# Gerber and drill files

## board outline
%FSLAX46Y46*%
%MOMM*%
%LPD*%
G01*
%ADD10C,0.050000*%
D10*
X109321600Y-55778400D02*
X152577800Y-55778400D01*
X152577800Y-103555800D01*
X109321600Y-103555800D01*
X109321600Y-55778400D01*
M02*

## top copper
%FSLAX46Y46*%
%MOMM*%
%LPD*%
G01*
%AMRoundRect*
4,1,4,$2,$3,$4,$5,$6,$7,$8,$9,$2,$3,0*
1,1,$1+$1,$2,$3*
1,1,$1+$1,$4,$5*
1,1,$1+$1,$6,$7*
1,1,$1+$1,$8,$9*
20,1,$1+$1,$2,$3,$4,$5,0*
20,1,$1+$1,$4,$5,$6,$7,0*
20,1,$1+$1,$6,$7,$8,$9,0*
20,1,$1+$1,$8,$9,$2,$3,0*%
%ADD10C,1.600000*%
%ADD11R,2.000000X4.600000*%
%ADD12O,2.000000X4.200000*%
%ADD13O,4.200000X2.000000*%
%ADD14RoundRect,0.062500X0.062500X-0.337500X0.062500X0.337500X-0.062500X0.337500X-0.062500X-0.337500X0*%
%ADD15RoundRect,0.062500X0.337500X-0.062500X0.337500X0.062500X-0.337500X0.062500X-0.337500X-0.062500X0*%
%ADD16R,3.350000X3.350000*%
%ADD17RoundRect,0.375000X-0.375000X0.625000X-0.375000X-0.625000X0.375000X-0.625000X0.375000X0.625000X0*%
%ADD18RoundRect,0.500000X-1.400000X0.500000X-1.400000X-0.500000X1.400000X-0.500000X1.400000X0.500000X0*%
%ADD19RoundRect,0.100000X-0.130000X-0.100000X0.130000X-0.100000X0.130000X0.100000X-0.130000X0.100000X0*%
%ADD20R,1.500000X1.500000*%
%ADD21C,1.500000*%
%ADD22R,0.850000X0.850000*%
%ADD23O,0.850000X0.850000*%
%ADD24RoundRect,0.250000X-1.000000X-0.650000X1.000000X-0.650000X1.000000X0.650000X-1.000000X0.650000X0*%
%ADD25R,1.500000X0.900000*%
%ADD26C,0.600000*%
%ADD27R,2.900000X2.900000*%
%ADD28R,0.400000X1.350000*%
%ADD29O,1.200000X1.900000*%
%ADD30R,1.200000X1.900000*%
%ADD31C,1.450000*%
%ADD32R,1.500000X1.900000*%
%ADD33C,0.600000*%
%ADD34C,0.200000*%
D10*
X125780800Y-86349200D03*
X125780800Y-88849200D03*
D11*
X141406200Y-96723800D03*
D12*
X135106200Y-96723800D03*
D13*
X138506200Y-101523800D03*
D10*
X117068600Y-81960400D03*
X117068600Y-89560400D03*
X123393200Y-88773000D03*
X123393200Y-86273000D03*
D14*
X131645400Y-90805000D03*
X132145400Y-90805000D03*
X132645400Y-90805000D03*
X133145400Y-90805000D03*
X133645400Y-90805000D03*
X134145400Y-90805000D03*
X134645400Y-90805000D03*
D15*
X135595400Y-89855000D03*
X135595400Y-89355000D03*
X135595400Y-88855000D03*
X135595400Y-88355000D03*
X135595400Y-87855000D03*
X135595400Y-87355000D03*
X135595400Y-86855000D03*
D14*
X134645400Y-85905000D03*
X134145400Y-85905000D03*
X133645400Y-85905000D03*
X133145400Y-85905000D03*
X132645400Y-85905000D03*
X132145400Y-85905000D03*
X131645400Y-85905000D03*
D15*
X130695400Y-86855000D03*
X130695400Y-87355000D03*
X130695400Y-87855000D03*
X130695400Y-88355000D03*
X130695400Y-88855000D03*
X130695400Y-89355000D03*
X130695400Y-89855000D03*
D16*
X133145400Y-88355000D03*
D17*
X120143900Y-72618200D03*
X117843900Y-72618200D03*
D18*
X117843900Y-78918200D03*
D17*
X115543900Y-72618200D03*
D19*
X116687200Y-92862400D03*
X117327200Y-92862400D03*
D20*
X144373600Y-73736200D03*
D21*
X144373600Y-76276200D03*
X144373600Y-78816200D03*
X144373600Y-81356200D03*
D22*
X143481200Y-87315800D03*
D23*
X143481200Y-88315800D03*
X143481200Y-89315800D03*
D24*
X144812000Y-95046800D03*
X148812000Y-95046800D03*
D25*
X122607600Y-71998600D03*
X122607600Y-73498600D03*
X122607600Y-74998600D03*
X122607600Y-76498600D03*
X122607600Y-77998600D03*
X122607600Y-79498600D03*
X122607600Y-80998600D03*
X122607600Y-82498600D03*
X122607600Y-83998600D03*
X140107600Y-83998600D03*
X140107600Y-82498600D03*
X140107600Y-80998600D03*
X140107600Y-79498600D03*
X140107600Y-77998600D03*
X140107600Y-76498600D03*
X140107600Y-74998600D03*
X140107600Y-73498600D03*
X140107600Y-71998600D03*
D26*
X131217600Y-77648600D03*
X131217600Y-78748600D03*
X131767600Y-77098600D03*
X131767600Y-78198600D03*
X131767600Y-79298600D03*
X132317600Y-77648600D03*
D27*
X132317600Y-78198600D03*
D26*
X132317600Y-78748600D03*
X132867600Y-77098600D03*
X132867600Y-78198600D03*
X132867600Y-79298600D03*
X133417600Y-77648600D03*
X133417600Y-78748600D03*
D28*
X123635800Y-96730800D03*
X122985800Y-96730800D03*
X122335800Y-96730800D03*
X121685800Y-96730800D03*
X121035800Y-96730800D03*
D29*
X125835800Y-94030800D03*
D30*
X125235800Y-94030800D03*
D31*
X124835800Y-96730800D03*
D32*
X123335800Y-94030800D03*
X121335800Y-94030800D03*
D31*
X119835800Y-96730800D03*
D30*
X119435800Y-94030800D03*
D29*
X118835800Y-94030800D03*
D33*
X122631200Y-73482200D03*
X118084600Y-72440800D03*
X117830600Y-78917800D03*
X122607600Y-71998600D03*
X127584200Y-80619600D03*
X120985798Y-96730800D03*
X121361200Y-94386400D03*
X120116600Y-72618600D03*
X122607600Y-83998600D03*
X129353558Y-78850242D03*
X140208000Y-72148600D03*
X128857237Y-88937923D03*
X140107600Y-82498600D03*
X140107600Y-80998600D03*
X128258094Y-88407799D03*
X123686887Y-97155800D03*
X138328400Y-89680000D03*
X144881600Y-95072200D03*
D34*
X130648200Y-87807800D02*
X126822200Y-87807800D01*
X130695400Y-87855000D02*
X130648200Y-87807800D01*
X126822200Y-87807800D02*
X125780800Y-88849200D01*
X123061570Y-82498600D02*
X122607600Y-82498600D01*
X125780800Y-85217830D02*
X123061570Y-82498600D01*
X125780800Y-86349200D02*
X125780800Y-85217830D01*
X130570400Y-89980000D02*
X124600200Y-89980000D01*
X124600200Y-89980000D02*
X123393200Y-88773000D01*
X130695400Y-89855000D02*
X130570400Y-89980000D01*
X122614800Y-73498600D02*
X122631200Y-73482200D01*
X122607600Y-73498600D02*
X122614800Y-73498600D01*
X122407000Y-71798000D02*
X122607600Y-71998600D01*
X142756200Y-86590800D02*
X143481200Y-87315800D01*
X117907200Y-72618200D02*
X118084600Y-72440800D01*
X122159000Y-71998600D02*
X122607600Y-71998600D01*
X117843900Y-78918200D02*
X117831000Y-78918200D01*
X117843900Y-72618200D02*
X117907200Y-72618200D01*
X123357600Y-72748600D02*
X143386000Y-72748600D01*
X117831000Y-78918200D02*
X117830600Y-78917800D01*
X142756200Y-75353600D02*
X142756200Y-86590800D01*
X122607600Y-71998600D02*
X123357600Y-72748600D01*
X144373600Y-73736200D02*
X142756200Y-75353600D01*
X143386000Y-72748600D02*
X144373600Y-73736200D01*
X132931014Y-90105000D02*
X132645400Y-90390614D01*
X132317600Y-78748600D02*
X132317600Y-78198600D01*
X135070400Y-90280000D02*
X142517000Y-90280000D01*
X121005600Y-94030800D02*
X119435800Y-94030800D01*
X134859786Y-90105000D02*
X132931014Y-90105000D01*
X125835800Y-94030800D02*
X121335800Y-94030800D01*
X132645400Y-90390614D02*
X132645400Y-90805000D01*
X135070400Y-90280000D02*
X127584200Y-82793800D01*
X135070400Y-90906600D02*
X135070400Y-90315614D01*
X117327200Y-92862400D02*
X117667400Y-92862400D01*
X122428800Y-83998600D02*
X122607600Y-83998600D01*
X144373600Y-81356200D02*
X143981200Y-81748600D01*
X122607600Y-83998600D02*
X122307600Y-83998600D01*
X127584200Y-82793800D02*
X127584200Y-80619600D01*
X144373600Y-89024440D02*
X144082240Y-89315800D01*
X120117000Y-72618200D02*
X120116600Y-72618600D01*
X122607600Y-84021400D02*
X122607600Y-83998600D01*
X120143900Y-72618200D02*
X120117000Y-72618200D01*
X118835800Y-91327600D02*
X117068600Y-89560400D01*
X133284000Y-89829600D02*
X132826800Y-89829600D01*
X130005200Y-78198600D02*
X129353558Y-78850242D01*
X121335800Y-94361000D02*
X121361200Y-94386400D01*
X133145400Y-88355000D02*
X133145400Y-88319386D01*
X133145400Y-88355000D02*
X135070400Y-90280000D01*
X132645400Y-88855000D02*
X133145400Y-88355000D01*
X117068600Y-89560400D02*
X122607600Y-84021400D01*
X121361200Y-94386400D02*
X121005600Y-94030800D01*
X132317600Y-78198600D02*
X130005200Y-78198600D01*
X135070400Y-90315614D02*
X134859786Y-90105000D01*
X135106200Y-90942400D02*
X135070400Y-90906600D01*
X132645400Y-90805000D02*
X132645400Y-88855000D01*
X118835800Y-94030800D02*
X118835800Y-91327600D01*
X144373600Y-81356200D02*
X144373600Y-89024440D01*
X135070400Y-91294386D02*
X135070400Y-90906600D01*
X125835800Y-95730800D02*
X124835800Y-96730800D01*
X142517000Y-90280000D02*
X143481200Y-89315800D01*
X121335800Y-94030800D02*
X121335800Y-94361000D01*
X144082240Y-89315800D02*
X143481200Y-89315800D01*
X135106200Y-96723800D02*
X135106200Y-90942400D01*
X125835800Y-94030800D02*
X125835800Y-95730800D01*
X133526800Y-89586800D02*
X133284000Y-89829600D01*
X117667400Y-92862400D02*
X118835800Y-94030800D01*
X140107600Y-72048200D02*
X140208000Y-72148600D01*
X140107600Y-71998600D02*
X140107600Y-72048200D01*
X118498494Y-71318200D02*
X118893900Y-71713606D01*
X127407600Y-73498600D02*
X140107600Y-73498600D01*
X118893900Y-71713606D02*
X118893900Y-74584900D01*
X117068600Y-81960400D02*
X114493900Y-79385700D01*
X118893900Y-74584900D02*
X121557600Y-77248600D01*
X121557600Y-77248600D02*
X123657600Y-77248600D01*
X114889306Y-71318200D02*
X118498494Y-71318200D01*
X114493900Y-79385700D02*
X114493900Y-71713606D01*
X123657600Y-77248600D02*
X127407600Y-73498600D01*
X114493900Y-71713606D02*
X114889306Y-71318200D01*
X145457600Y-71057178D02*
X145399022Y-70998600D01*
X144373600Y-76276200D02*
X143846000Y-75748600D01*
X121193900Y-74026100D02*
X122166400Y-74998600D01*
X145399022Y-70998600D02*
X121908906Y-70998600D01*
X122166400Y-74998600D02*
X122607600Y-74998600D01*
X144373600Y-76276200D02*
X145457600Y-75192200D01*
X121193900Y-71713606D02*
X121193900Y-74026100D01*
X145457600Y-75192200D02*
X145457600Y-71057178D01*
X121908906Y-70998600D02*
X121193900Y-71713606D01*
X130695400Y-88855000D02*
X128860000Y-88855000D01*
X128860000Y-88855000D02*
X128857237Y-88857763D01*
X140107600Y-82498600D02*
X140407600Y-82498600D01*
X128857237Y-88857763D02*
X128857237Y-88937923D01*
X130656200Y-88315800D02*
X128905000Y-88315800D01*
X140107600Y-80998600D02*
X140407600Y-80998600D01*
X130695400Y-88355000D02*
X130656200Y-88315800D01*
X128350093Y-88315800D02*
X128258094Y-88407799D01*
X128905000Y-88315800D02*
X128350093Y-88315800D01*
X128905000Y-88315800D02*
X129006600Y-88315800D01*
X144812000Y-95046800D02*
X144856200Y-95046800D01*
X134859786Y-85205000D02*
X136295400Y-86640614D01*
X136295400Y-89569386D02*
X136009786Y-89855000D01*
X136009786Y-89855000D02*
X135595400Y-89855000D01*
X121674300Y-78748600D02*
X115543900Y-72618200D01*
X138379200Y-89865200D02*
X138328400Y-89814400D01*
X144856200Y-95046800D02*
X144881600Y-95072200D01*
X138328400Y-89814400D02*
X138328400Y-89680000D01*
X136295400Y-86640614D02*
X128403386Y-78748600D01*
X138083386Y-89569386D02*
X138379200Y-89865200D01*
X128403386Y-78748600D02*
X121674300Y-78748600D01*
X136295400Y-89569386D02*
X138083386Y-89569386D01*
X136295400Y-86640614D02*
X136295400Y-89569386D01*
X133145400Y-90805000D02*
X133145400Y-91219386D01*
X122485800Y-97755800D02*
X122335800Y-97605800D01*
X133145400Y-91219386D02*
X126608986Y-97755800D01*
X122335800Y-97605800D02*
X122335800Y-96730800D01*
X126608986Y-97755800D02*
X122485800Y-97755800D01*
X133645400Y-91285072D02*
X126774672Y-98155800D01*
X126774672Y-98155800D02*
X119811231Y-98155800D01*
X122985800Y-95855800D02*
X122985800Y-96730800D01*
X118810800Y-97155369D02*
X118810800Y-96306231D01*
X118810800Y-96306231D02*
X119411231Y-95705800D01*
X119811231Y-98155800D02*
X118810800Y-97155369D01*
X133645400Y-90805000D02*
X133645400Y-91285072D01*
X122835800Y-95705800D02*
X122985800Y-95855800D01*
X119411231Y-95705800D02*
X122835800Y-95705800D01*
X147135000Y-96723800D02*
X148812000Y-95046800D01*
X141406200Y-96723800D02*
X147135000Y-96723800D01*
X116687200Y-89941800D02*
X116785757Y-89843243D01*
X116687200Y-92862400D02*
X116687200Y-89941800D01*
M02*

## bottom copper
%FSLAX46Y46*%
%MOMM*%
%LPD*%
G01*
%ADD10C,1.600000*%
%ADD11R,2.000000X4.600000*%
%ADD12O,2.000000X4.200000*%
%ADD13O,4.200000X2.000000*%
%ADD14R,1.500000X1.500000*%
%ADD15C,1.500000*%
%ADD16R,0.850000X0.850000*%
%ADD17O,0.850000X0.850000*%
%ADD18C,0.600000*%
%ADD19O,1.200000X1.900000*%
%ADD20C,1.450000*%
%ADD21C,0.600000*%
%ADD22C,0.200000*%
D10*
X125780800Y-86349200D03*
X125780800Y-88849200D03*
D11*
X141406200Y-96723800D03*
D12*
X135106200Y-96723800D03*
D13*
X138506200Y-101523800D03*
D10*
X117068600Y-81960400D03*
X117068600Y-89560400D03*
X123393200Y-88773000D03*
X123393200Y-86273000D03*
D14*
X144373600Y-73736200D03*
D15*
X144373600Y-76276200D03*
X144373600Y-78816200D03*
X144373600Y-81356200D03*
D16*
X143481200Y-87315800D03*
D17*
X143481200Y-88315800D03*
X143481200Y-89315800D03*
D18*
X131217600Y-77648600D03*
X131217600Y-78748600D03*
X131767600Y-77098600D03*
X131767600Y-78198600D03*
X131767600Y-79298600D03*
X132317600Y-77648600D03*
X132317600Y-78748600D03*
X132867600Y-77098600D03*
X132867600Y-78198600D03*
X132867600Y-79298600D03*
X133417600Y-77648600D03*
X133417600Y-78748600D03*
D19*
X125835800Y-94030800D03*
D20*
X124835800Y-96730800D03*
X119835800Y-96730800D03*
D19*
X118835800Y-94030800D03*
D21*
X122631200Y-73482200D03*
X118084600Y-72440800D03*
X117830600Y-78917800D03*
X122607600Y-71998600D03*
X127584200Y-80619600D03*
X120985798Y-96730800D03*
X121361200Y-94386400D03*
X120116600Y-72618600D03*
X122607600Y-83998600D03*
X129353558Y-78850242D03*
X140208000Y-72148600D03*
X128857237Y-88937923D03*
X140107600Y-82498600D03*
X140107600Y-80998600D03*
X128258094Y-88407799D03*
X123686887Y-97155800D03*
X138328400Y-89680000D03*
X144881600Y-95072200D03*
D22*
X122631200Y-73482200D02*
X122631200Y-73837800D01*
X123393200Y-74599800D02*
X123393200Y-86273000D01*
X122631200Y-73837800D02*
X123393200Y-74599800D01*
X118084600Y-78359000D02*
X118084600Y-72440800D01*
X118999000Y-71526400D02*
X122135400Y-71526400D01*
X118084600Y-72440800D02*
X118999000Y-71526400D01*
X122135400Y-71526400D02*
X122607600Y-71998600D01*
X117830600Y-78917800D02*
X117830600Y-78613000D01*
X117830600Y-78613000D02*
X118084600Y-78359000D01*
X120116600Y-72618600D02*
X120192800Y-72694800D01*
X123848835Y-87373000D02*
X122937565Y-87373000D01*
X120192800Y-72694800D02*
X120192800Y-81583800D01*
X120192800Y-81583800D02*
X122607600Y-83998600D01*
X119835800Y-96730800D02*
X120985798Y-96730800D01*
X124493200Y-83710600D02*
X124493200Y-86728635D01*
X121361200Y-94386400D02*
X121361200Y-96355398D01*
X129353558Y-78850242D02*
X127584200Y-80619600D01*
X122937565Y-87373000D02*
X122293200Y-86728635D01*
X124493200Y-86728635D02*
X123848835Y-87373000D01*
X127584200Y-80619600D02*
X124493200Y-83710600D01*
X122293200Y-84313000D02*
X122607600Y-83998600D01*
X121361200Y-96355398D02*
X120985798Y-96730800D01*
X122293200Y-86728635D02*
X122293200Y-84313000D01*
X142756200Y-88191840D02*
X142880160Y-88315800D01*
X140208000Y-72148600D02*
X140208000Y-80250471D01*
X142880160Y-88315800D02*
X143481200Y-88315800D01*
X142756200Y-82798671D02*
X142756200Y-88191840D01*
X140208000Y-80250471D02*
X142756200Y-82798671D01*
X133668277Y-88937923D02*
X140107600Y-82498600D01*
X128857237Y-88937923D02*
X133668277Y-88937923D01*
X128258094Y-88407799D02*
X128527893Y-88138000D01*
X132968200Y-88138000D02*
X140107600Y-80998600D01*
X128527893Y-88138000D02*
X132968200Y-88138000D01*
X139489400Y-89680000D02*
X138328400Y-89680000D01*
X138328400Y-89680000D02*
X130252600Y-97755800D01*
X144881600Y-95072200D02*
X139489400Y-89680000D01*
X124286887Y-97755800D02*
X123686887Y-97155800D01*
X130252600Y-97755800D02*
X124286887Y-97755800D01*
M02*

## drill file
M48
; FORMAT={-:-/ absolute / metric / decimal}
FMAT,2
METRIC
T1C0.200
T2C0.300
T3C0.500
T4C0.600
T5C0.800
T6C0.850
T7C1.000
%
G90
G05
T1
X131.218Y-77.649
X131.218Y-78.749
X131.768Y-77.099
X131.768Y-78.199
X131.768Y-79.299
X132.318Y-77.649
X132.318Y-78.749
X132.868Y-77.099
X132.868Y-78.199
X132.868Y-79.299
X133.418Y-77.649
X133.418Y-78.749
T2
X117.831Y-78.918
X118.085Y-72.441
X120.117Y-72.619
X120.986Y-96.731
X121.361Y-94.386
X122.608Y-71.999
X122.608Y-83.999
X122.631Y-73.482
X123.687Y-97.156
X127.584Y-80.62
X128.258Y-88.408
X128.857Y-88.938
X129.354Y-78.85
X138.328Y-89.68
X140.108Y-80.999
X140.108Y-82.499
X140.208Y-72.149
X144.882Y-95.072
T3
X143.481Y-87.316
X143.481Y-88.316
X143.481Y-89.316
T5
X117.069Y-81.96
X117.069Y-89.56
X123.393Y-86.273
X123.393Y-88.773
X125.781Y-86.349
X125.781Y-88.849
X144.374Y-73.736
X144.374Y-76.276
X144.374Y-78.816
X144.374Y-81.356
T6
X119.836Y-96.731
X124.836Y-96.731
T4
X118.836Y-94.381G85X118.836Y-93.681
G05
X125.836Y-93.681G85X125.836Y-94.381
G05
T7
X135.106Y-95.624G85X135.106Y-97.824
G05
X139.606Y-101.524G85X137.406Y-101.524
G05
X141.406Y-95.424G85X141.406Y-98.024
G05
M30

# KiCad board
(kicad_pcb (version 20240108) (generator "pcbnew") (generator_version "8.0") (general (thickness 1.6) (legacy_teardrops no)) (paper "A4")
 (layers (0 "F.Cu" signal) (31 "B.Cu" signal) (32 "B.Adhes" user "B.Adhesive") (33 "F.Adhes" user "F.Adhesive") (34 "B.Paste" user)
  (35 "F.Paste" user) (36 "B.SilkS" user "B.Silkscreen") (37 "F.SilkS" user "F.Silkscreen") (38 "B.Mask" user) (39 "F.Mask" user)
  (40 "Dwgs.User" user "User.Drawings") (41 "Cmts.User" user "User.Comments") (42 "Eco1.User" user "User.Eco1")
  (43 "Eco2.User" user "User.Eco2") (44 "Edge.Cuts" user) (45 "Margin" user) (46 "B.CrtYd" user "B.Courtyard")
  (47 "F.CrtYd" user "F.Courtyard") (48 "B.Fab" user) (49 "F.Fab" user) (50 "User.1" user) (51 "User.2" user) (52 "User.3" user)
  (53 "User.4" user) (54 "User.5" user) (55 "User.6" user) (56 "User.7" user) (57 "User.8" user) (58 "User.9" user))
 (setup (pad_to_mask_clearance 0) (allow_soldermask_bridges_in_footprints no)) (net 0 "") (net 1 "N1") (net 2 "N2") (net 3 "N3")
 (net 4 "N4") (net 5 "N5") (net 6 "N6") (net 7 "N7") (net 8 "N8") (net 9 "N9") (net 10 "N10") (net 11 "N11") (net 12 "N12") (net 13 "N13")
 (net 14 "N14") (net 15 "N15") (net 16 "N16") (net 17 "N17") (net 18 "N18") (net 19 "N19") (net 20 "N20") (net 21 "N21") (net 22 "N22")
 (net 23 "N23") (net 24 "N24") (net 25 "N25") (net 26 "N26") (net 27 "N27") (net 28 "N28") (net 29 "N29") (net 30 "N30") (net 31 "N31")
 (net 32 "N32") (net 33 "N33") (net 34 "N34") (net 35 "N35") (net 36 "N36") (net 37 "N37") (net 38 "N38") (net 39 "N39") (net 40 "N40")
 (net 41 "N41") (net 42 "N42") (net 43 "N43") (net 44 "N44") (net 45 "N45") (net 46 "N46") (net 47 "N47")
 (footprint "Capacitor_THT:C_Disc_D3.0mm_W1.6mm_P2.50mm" (layer "F.Cu") (at 125.7808 86.3492 -90)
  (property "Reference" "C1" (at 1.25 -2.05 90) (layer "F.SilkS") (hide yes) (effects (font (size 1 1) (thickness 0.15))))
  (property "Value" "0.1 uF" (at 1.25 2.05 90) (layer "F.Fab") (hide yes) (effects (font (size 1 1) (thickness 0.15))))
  (pad "1" thru_hole circle (at 0 0 270) (size 1.6 1.6) (drill 0.8) (layers "*.Cu" "*.Mask") (remove_unused_layers no) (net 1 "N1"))
  (pad "2" thru_hole circle (at 2.5 0 270) (size 1.6 1.6) (drill 0.8) (layers "*.Cu" "*.Mask") (remove_unused_layers no) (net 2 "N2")))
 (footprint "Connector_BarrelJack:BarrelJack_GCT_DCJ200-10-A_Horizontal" (layer "F.Cu") (at 141.4062 96.7238 -90)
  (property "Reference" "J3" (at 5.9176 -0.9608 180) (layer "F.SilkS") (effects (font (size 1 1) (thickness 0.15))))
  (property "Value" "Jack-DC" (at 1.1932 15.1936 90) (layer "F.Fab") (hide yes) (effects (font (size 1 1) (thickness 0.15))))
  (pad "1" thru_hole rect (at 0 0 270) (size 4.6 2) (drill oval 3.6 1) (layers "*.Cu" "*.Mask") (remove_unused_layers no) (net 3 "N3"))
  (pad "2" thru_hole oval (at 0 6.3 270) (size 4.2 2) (drill oval 3.2 1) (layers "*.Cu" "*.Mask") (remove_unused_layers no) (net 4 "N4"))
  (pad "3" thru_hole oval (at 4.8 2.9 270) (size 2 4.2) (drill oval 1 3.2) (layers "*.Cu" "*.Mask") (remove_unused_layers no)))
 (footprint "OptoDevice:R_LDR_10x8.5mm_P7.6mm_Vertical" (layer "F.Cu") (at 117.0686 81.9604 -90)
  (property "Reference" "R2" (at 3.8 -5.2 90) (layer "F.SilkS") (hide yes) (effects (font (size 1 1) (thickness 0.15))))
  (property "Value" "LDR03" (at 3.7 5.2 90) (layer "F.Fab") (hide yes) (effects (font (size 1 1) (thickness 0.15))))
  (pad "1" thru_hole circle (at 0 0 270) (size 1.6 1.6) (drill 0.8) (layers "*.Cu" "*.Mask") (remove_unused_layers no) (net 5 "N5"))
  (pad "2" thru_hole circle (at 7.6 0 270) (size 1.6 1.6) (drill 0.8) (layers "*.Cu" "*.Mask") (remove_unused_layers no) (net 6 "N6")))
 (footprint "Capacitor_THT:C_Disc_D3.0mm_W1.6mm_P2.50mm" (layer "F.Cu") (at 123.3932 88.773 90)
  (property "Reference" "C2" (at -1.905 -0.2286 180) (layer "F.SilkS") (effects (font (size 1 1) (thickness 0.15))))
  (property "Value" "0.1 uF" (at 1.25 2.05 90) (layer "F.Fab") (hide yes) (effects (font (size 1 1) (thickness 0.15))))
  (pad "1" thru_hole circle (at 0 0 90) (size 1.6 1.6) (drill 0.8) (layers "*.Cu" "*.Mask") (remove_unused_layers no) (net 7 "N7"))
  (pad "2" thru_hole circle (at 2.5 0 90) (size 1.6 1.6) (drill 0.8) (layers "*.Cu" "*.Mask") (remove_unused_layers no) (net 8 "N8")))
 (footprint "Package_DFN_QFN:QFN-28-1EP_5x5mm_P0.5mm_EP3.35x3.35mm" (layer "F.Cu") (at 133.1454 88.355 90)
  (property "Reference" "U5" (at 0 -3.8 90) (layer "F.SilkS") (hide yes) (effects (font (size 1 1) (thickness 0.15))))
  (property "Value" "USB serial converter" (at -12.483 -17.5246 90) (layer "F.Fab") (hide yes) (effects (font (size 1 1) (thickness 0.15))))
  (pad "" smd roundrect (at -1.12 -1.12 90) (size 0.9 0.9) (layers "F.Paste") (roundrect_rratio 0.25))
  (pad "" smd roundrect (at -1.12 0 90) (size 0.9 0.9) (layers "F.Paste") (roundrect_rratio 0.25))
  (pad "" smd roundrect (at -1.12 1.12 90) (size 0.9 0.9) (layers "F.Paste") (roundrect_rratio 0.25))
  (pad "" smd roundrect (at 0 -1.12 90) (size 0.9 0.9) (layers "F.Paste") (roundrect_rratio 0.25))
  (pad "" smd roundrect (at 0 0 90) (size 0.9 0.9) (layers "F.Paste") (roundrect_rratio 0.25))
  (pad "" smd roundrect (at 0 1.12 90) (size 0.9 0.9) (layers "F.Paste") (roundrect_rratio 0.25))
  (pad "" smd roundrect (at 1.12 -1.12 90) (size 0.9 0.9) (layers "F.Paste") (roundrect_rratio 0.25))
  (pad "" smd roundrect (at 1.12 0 90) (size 0.9 0.9) (layers "F.Paste") (roundrect_rratio 0.25))
  (pad "" smd roundrect (at 1.12 1.12 90) (size 0.9 0.9) (layers "F.Paste") (roundrect_rratio 0.25))
  (pad "1" smd roundrect (at -2.45 -1.5 90) (size 0.8 0.25) (layers "F.Cu" "F.Paste" "F.Mask") (roundrect_rratio 0.25) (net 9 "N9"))
  (pad "2" smd roundrect (at -2.45 -1 90) (size 0.8 0.25) (layers "F.Cu" "F.Paste" "F.Mask") (roundrect_rratio 0.25) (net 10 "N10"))
  (pad "3" smd roundrect (at -2.45 -0.5 90) (size 0.8 0.25) (layers "F.Cu" "F.Paste" "F.Mask") (roundrect_rratio 0.25) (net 4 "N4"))
  (pad "4" smd roundrect (at -2.45 0 90) (size 0.8 0.25) (layers "F.Cu" "F.Paste" "F.Mask") (roundrect_rratio 0.25) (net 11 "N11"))
  (pad "5" smd roundrect (at -2.45 0.5 90) (size 0.8 0.25) (layers "F.Cu" "F.Paste" "F.Mask") (roundrect_rratio 0.25) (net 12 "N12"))
  (pad "6" smd roundrect (at -2.45 1 90) (size 0.8 0.25) (layers "F.Cu" "F.Paste" "F.Mask") (roundrect_rratio 0.25) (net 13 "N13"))
  (pad "7" smd roundrect (at -2.45 1.5 90) (size 0.8 0.25) (layers "F.Cu" "F.Paste" "F.Mask") (roundrect_rratio 0.25) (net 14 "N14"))
  (pad "8" smd roundrect (at -1.5 2.45 90) (size 0.25 0.8) (layers "F.Cu" "F.Paste" "F.Mask") (roundrect_rratio 0.25) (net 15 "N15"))
  (pad "9" smd roundrect (at -1 2.45 90) (size 0.25 0.8) (layers "F.Cu" "F.Paste" "F.Mask") (roundrect_rratio 0.25) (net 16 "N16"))
  (pad "10" smd roundrect (at -0.5 2.45 90) (size 0.25 0.8) (layers "F.Cu" "F.Paste" "F.Mask") (roundrect_rratio 0.25) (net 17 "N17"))
  (pad "11" smd roundrect (at 0 2.45 90) (size 0.25 0.8) (layers "F.Cu" "F.Paste" "F.Mask") (roundrect_rratio 0.25) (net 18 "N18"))
  (pad "12" smd roundrect (at 0.5 2.45 90) (size 0.25 0.8) (layers "F.Cu" "F.Paste" "F.Mask") (roundrect_rratio 0.25) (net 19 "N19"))
  (pad "13" smd roundrect (at 1 2.45 90) (size 0.25 0.8) (layers "F.Cu" "F.Paste" "F.Mask") (roundrect_rratio 0.25) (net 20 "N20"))
  (pad "14" smd roundrect (at 1.5 2.45 90) (size 0.25 0.8) (layers "F.Cu" "F.Paste" "F.Mask") (roundrect_rratio 0.25) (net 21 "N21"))
  (pad "15" smd roundrect (at 2.45 1.5 90) (size 0.8 0.25) (layers "F.Cu" "F.Paste" "F.Mask") (roundrect_rratio 0.25) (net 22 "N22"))
  (pad "16" smd roundrect (at 2.45 1 90) (size 0.8 0.25) (layers "F.Cu" "F.Paste" "F.Mask") (roundrect_rratio 0.25) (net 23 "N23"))
  (pad "17" smd roundrect (at 2.45 0.5 90) (size 0.8 0.25) (layers "F.Cu" "F.Paste" "F.Mask") (roundrect_rratio 0.25) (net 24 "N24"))
  (pad "18" smd roundrect (at 2.45 0 90) (size 0.8 0.25) (layers "F.Cu" "F.Paste" "F.Mask") (roundrect_rratio 0.25) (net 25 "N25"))
  (pad "19" smd roundrect (at 2.45 -0.5 90) (size 0.8 0.25) (layers "F.Cu" "F.Paste" "F.Mask") (roundrect_rratio 0.25) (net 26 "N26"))
  (pad "20" smd roundrect (at 2.45 -1 90) (size 0.8 0.25) (layers "F.Cu" "F.Paste" "F.Mask") (roundrect_rratio 0.25) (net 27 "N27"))
  (pad "21" smd roundrect (at 2.45 -1.5 90) (size 0.8 0.25) (layers "F.Cu" "F.Paste" "F.Mask") (roundrect_rratio 0.25) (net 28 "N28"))
  (pad "22" smd roundrect (at 1.5 -2.45 90) (size 0.25 0.8) (layers "F.Cu" "F.Paste" "F.Mask") (roundrect_rratio 0.25) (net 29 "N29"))
  (pad "23" smd roundrect (at 1 -2.45 90) (size 0.25 0.8) (layers "F.Cu" "F.Paste" "F.Mask") (roundrect_rratio 0.25) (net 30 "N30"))
  (pad "24" smd roundrect (at 0.5 -2.45 90) (size 0.25 0.8) (layers "F.Cu" "F.Paste" "F.Mask") (roundrect_rratio 0.25) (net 2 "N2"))
  (pad "25" smd roundrect (at 0 -2.45 90) (size 0.25 0.8) (layers "F.Cu" "F.Paste" "F.Mask") (roundrect_rratio 0.25) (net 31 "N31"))
  (pad "26" smd roundrect (at -0.5 -2.45 90) (size 0.25 0.8) (layers "F.Cu" "F.Paste" "F.Mask") (roundrect_rratio 0.25) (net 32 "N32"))
  (pad "27" smd roundrect (at -1 -2.45 90) (size 0.25 0.8) (layers "F.Cu" "F.Paste" "F.Mask") (roundrect_rratio 0.25) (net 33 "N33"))
  (pad "28" smd roundrect (at -1.5 -2.45 90) (size 0.25 0.8) (layers "F.Cu" "F.Paste" "F.Mask") (roundrect_rratio 0.25) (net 7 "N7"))
  (pad "29" smd rect (at 0 0 90) (size 3.35 3.35) (layers "F.Cu" "F.Mask") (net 4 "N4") (zone_connect 2)))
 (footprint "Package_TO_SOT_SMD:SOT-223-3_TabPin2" (layer "F.Cu") (at 117.8439 75.7682 -90)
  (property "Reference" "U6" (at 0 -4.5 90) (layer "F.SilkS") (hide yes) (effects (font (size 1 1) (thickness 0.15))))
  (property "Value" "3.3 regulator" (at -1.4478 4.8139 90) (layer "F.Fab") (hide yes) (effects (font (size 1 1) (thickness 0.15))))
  (pad "1" smd roundrect (at -3.15 -2.3 270) (size 2 1.5) (layers "F.Cu" "F.Paste" "F.Mask") (roundrect_rratio 0.25) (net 4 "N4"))
  (pad "2" smd roundrect (at -3.15 0 270) (size 2 1.5) (layers "F.Cu" "F.Paste" "F.Mask") (roundrect_rratio 0.25) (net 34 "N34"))
  (pad "2" smd roundrect (at 3.15 0 270) (size 2 3.8) (layers "F.Cu" "F.Paste" "F.Mask") (roundrect_rratio 0.25) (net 34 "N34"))
  (pad "3" smd roundrect (at -3.15 2.3 270) (size 2 1.5) (layers "F.Cu" "F.Paste" "F.Mask") (roundrect_rratio 0.25) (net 15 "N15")))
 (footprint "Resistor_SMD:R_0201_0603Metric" (layer "F.Cu") (at 117.0072 92.8624)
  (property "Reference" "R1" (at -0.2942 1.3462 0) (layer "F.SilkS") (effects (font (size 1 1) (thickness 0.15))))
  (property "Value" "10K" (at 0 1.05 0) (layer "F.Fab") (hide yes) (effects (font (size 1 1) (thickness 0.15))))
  (pad "" smd roundrect (at -0.345 0) (size 0.318 0.36) (layers "F.Paste") (roundrect_rratio 0.25))
  (pad "" smd roundrect (at 0.345 0) (size 0.318 0.36) (layers "F.Paste") (roundrect_rratio 0.25))
  (pad "1" smd roundrect (at -0.32 0) (size 0.46 0.4) (layers "F.Cu" "F.Mask") (roundrect_rratio 0.25) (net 6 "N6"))
  (pad "2" smd roundrect (at 0.32 0) (size 0.46 0.4) (layers "F.Cu" "F.Mask") (roundrect_rratio 0.25) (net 4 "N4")))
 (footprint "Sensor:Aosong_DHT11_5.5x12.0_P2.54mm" (layer "F.Cu") (at 144.3736 73.7362)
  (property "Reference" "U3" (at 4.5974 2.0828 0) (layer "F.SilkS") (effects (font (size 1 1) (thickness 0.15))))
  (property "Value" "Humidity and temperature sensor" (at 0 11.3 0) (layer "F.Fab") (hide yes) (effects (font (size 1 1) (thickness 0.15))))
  (pad "1" thru_hole rect (at 0 0) (size 1.5 1.5) (drill 0.8) (layers "*.Cu" "*.Mask") (remove_unused_layers no) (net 34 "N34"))
  (pad "2" thru_hole circle (at 0 2.54) (size 1.5 1.5) (drill 0.8) (layers "*.Cu" "*.Mask") (remove_unused_layers no) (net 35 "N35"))
  (pad "3" thru_hole circle (at 0 5.08) (size 1.5 1.5) (drill 0.8) (layers "*.Cu" "*.Mask") (remove_unused_layers no) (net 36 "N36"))
  (pad "4" thru_hole circle (at 0 7.62) (size 1.5 1.5) (drill 0.8) (layers "*.Cu" "*.Mask") (remove_unused_layers no) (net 4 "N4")))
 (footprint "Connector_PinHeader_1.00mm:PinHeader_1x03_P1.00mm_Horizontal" (layer "F.Cu") (at 143.4812 87.3158)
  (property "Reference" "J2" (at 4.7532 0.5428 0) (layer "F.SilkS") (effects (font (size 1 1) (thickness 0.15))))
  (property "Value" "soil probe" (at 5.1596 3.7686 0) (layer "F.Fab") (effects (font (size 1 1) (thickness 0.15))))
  (pad "1" thru_hole rect (at 0 0) (size 0.85 0.85) (drill 0.5) (layers "*.Cu" "*.Mask") (remove_unused_layers no) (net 34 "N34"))
  (pad "2" thru_hole oval (at 0 1) (size 0.85 0.85) (drill 0.5) (layers "*.Cu" "*.Mask") (remove_unused_layers no) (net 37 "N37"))
  (pad "3" thru_hole oval (at 0 2) (size 0.85 0.85) (drill 0.5) (layers "*.Cu" "*.Mask") (remove_unused_layers no) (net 4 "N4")))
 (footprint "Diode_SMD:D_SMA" (layer "F.Cu") (at 146.812 95.0468)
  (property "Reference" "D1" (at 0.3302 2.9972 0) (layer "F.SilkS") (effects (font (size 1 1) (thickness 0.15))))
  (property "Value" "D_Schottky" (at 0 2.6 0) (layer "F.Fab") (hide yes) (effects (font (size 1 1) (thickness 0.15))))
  (pad "1" smd roundrect (at -2 0) (size 2.5 1.8) (layers "F.Cu" "F.Paste" "F.Mask") (roundrect_rratio 0.1388888889) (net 15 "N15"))
  (pad "2" smd roundrect (at 2 0) (size 2.5 1.8) (layers "F.Cu" "F.Paste" "F.Mask") (roundrect_rratio 0.1388888889) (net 3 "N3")))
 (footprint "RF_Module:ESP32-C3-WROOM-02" (layer "F.Cu") (at 131.3576 77.9986)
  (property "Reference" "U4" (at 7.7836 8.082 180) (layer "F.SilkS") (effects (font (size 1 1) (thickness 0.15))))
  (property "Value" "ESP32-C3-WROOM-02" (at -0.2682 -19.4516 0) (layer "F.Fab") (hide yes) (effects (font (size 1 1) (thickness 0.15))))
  (pad "" smd rect (at -0.14 -0.9) (size 0.7 0.7) (layers "F.Paste"))
  (pad "" smd rect (at -0.14 0.2) (size 0.7 0.7) (layers "F.Paste"))
  (pad "" smd rect (at -0.14 1.3) (size 0.7 0.7) (layers "F.Paste"))
  (pad "" smd rect (at 0.96 -0.9) (size 0.7 0.7) (layers "F.Paste"))
  (pad "" smd rect (at 0.96 0.2) (size 0.7 0.7) (layers "F.Paste"))
  (pad "" smd rect (at 0.96 1.3) (size 0.7 0.7) (layers "F.Paste"))
  (pad "" smd rect (at 2.06 -0.9) (size 0.7 0.7) (layers "F.Paste"))
  (pad "" smd rect (at 2.06 0.2) (size 0.7 0.7) (layers "F.Paste"))
  (pad "" smd rect (at 2.06 1.3) (size 0.7 0.7) (layers "F.Paste"))
  (pad "1" smd rect (at -8.75 -6) (size 1.5 0.9) (layers "F.Cu" "F.Paste" "F.Mask") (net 34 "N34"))
  (pad "2" smd rect (at -8.75 -4.5) (size 1.5 0.9) (layers "F.Cu" "F.Paste" "F.Mask") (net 8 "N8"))
  (pad "3" smd rect (at -8.75 -3) (size 1.5 0.9) (layers "F.Cu" "F.Paste" "F.Mask") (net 35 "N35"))
  (pad "4" smd rect (at -8.75 -1.5) (size 1.5 0.9) (layers "F.Cu" "F.Paste" "F.Mask") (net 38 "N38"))
  (pad "5" smd rect (at -8.75 0) (size 1.5 0.9) (layers "F.Cu" "F.Paste" "F.Mask") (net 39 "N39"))
  (pad "6" smd rect (at -8.75 1.5) (size 1.5 0.9) (layers "F.Cu" "F.Paste" "F.Mask") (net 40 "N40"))
  (pad "7" smd rect (at -8.75 3) (size 1.5 0.9) (layers "F.Cu" "F.Paste" "F.Mask") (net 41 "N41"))
  (pad "8" smd rect (at -8.75 4.5) (size 1.5 0.9) (layers "F.Cu" "F.Paste" "F.Mask") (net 1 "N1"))
  (pad "9" smd rect (at -8.75 6) (size 1.5 0.9) (layers "F.Cu" "F.Paste" "F.Mask") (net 4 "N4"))
  (pad "10" smd rect (at 8.75 6) (size 1.5 0.9) (layers "F.Cu" "F.Paste" "F.Mask") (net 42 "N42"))
  (pad "11" smd rect (at 8.75 4.5) (size 1.5 0.9) (layers "F.Cu" "F.Paste" "F.Mask") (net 32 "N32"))
  (pad "12" smd rect (at 8.75 3) (size 1.5 0.9) (layers "F.Cu" "F.Paste" "F.Mask") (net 31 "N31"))
  (pad "13" smd rect (at 8.75 1.5) (size 1.5 0.9) (layers "F.Cu" "F.Paste" "F.Mask") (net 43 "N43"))
  (pad "14" smd rect (at 8.75 0) (size 1.5 0.9) (layers "F.Cu" "F.Paste" "F.Mask") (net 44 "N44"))
  (pad "15" smd rect (at 8.75 -1.5) (size 1.5 0.9) (layers "F.Cu" "F.Paste" "F.Mask") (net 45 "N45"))
  (pad "16" smd rect (at 8.75 -3) (size 1.5 0.9) (layers "F.Cu" "F.Paste" "F.Mask") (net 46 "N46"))
  (pad "17" smd rect (at 8.75 -4.5) (size 1.5 0.9) (layers "F.Cu" "F.Paste" "F.Mask") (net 5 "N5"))
  (pad "18" smd rect (at 8.75 -6) (size 1.5 0.9) (layers "F.Cu" "F.Paste" "F.Mask") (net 37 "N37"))
  (pad "19" thru_hole circle (at -0.14 -0.35) (size 0.6 0.6) (drill 0.2) (layers "*.Cu" "F.Mask") (remove_unused_layers no) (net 4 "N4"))
  (pad "19" thru_hole circle (at -0.14 0.75) (size 0.6 0.6) (drill 0.2) (layers "*.Cu" "F.Mask") (remove_unused_layers no) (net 4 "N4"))
  (pad "19" thru_hole circle (at 0.41 -0.9) (size 0.6 0.6) (drill 0.2) (layers "*.Cu" "F.Mask") (remove_unused_layers no) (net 4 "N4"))
  (pad "19" thru_hole circle (at 0.41 0.2) (size 0.6 0.6) (drill 0.2) (layers "*.Cu" "F.Mask") (remove_unused_layers no) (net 4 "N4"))
  (pad "19" thru_hole circle (at 0.41 1.3) (size 0.6 0.6) (drill 0.2) (layers "*.Cu" "F.Mask") (remove_unused_layers no) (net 4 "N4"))
  (pad "19" thru_hole circle (at 0.96 -0.35) (size 0.6 0.6) (drill 0.2) (layers "*.Cu" "F.Mask") (remove_unused_layers no) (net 4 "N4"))
  (pad "19" smd rect (at 0.96 0.2) (size 2.9 2.9) (layers "F.Cu" "F.Mask") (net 4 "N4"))
  (pad "19" thru_hole circle (at 0.96 0.75) (size 0.6 0.6) (drill 0.2) (layers "*.Cu" "F.Mask") (remove_unused_layers no) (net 4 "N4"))
  (pad "19" thru_hole circle (at 1.51 -0.9) (size 0.6 0.6) (drill 0.2) (layers "*.Cu" "F.Mask") (remove_unused_layers no) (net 4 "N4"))
  (pad "19" thru_hole circle (at 1.51 0.2) (size 0.6 0.6) (drill 0.2) (layers "*.Cu" "F.Mask") (remove_unused_layers no) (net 4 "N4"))
  (pad "19" thru_hole circle (at 1.51 1.3) (size 0.6 0.6) (drill 0.2) (layers "*.Cu" "F.Mask") (remove_unused_layers no) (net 4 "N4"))
  (pad "19" thru_hole circle (at 2.06 -0.35) (size 0.6 0.6) (drill 0.2) (layers "*.Cu" "F.Mask") (remove_unused_layers no) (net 4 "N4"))
  (pad "19" thru_hole circle (at 2.06 0.75) (size 0.6 0.6) (drill 0.2) (layers "*.Cu" "F.Mask") (remove_unused_layers no) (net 4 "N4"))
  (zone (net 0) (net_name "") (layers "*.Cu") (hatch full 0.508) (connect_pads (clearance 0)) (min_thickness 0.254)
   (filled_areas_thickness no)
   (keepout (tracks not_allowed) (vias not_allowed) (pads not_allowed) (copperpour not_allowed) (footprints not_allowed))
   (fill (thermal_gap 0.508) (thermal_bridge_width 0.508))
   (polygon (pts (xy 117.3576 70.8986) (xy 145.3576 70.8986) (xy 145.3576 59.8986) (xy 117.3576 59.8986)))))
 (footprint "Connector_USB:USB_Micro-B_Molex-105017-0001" (layer "F.Cu") (at 122.3358 95.2683 180)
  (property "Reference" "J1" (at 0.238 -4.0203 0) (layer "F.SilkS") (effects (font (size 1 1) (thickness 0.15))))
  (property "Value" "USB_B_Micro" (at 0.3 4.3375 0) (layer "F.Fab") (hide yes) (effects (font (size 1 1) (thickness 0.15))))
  (pad "1" smd rect (at -1.3 -1.4625 180) (size 0.4 1.35) (layers "F.Cu" "F.Paste" "F.Mask") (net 15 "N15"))
  (pad "2" smd rect (at -0.65 -1.4625 180) (size 0.4 1.35) (layers "F.Cu" "F.Paste" "F.Mask") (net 12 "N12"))
  (pad "3" smd rect (at 0 -1.4625 180) (size 0.4 1.35) (layers "F.Cu" "F.Paste" "F.Mask") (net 11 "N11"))
  (pad "4" smd rect (at 0.65 -1.4625 180) (size 0.4 1.35) (layers "F.Cu" "F.Paste" "F.Mask") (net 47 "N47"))
  (pad "5" smd rect (at 1.3 -1.4625 180) (size 0.4 1.35) (layers "F.Cu" "F.Paste" "F.Mask") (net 4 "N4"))
  (pad "6" thru_hole oval (at -3.5 1.2375) (size 1.2 1.9) (drill oval 0.6 1.3) (layers "*.Cu" "*.Mask") (remove_unused_layers no)
   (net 4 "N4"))
  (pad "6" smd rect (at -2.9 1.2375 180) (size 1.2 1.9) (layers "F.Cu" "F.Mask") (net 4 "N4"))
  (pad "6" thru_hole circle (at -2.5 -1.4625 180) (size 1.45 1.45) (drill 0.85) (layers "*.Cu" "*.Mask") (remove_unused_layers no)
   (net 4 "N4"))
  (pad "6" smd rect (at -1 1.2375 180) (size 1.5 1.9) (layers "F.Cu" "F.Paste" "F.Mask") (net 4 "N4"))
  (pad "6" smd rect (at 1 1.2375 180) (size 1.5 1.9) (layers "F.Cu" "F.Paste" "F.Mask") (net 4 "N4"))
  (pad "6" thru_hole circle (at 2.5 -1.4625 180) (size 1.45 1.45) (drill 0.85) (layers "*.Cu" "*.Mask") (remove_unused_layers no)
   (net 4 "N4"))
  (pad "6" smd rect (at 2.9 1.2375 180) (size 1.2 1.9) (layers "F.Cu" "F.Mask") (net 4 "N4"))
  (pad "6" thru_hole oval (at 3.5 1.2375 180) (size 1.2 1.9) (drill oval 0.6 1.3) (layers "*.Cu" "*.Mask") (remove_unused_layers no)
   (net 4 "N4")))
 (gr_rect (start 109.3216 55.7784) (end 152.5778 103.5558) (stroke (width 0.05) (type default)) (fill none) (layer "Edge.Cuts"))
 (segment (start 130.6482 87.8078) (end 126.8222 87.8078) (width 0.2) (layer "F.Cu") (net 2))
 (segment (start 130.6954 87.855) (end 130.6482 87.8078) (width 0.2) (layer "F.Cu") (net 2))
 (segment (start 126.8222 87.8078) (end 125.7808 88.8492) (width 0.2) (layer "F.Cu") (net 2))
 (segment (start 123.06157 82.4986) (end 122.6076 82.4986) (width 0.2) (layer "F.Cu") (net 1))
 (segment (start 125.7808 85.21783) (end 123.06157 82.4986) (width 0.2) (layer "F.Cu") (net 1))
 (segment (start 125.7808 86.3492) (end 125.7808 85.21783) (width 0.2) (layer "F.Cu") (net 1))
 (segment (start 130.5704 89.98) (end 124.6002 89.98) (width 0.2) (layer "F.Cu") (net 7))
 (segment (start 124.6002 89.98) (end 123.3932 88.773) (width 0.2) (layer "F.Cu") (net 7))
 (segment (start 130.6954 89.855) (end 130.5704 89.98) (width 0.2) (layer "F.Cu") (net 7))
 (segment (start 122.6148 73.4986) (end 122.6312 73.4822) (width 0.2) (layer "F.Cu") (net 8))
 (segment (start 122.6076 73.4986) (end 122.6148 73.4986) (width 0.2) (layer "F.Cu") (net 8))
 (via (at 122.6312 73.4822) (size 0.6) (drill 0.3) (layers "F.Cu" "B.Cu") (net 8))
 (segment (start 122.6312 73.4822) (end 122.6312 73.8378) (width 0.2) (layer "B.Cu") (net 8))
 (segment (start 123.3932 74.5998) (end 123.3932 86.273) (width 0.2) (layer "B.Cu") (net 8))
 (segment (start 122.6312 73.8378) (end 123.3932 74.5998) (width 0.2) (layer "B.Cu") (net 8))
 (segment (start 122.407 71.798) (end 122.6076 71.9986) (width 0.2) (layer "F.Cu") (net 34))
 (segment (start 142.7562 86.5908) (end 143.4812 87.3158) (width 0.2) (layer "F.Cu") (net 34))
 (segment (start 117.9072 72.6182) (end 118.0846 72.4408) (width 0.2) (layer "F.Cu") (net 34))
 (segment (start 122.159 71.9986) (end 122.6076 71.9986) (width 0.2) (layer "F.Cu") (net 34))
 (segment (start 117.8439 78.9182) (end 117.831 78.9182) (width 0.2) (layer "F.Cu") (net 34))
 (segment (start 117.8439 72.6182) (end 117.9072 72.6182) (width 0.2) (layer "F.Cu") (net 34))
 (segment (start 123.3576 72.7486) (end 143.386 72.7486) (width 0.2) (layer "F.Cu") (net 34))
 (segment (start 117.831 78.9182) (end 117.8306 78.9178) (width 0.2) (layer "F.Cu") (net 34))
 (segment (start 142.7562 75.3536) (end 142.7562 86.5908) (width 0.2) (layer "F.Cu") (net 34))
 (segment (start 122.6076 71.9986) (end 123.3576 72.7486) (width 0.2) (layer "F.Cu") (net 34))
 (segment (start 144.3736 73.7362) (end 142.7562 75.3536) (width 0.2) (layer "F.Cu") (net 34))
 (segment (start 143.386 72.7486) (end 144.3736 73.7362) (width 0.2) (layer "F.Cu") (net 34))
 (via (at 118.0846 72.4408) (size 0.6) (drill 0.3) (layers "F.Cu" "B.Cu") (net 34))
 (via (at 117.8306 78.9178) (size 0.6) (drill 0.3) (layers "F.Cu" "B.Cu") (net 34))
 (via (at 122.6076 71.9986) (size 0.6) (drill 0.3) (layers "F.Cu" "B.Cu") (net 34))
 (segment (start 118.0846 78.359) (end 118.0846 72.4408) (width 0.2) (layer "B.Cu") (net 34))
 (segment (start 118.999 71.5264) (end 122.1354 71.5264) (width 0.2) (layer "B.Cu") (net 34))
 (segment (start 118.0846 72.4408) (end 118.999 71.5264) (width 0.2) (layer "B.Cu") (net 34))
 (segment (start 122.1354 71.5264) (end 122.6076 71.9986) (width 0.2) (layer "B.Cu") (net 34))
 (segment (start 117.8306 78.9178) (end 117.8306 78.613) (width 0.2) (layer "B.Cu") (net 34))
 (segment (start 117.8306 78.613) (end 118.0846 78.359) (width 0.2) (layer "B.Cu") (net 34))
 (segment (start 132.931014 90.105) (end 132.6454 90.390614) (width 0.2) (layer "F.Cu") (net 4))
 (segment (start 132.3176 78.7486) (end 132.3176 78.1986) (width 0.2) (layer "F.Cu") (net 4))
 (segment (start 135.0704 90.28) (end 142.517 90.28) (width 0.2) (layer "F.Cu") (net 4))
 (segment (start 121.0056 94.0308) (end 119.4358 94.0308) (width 0.2) (layer "F.Cu") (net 4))
 (segment (start 134.859786 90.105) (end 132.931014 90.105) (width 0.2) (layer "F.Cu") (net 4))
 (segment (start 125.8358 94.0308) (end 121.3358 94.0308) (width 0.2) (layer "F.Cu") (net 4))
 (segment (start 132.6454 90.390614) (end 132.6454 90.805) (width 0.2) (layer "F.Cu") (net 4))
 (segment (start 135.0704 90.28) (end 127.5842 82.7938) (width 0.2) (layer "F.Cu") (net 4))
 (segment (start 135.0704 90.9066) (end 135.0704 90.315614) (width 0.2) (layer "F.Cu") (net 4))
 (segment (start 117.3272 92.8624) (end 117.6674 92.8624) (width 0.2) (layer "F.Cu") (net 4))
 (segment (start 122.4288 83.9986) (end 122.6076 83.9986) (width 0.2) (layer "F.Cu") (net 4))
 (segment (start 144.3736 81.3562) (end 143.9812 81.7486) (width 0.2) (layer "F.Cu") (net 4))
 (segment (start 122.6076 83.9986) (end 122.3076 83.9986) (width 0.2) (layer "F.Cu") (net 4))
 (segment (start 127.5842 82.7938) (end 127.5842 80.6196) (width 0.2) (layer "F.Cu") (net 4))
 (segment (start 144.3736 89.02444) (end 144.08224 89.3158) (width 0.2) (layer "F.Cu") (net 4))
 (segment (start 120.117 72.6182) (end 120.1166 72.6186) (width 0.2) (layer "F.Cu") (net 4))
 (segment (start 122.6076 84.0214) (end 122.6076 83.9986) (width 0.2) (layer "F.Cu") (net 4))
 (segment (start 120.1439 72.6182) (end 120.117 72.6182) (width 0.2) (layer "F.Cu") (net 4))
 (segment (start 118.8358 91.3276) (end 117.0686 89.5604) (width 0.2) (layer "F.Cu") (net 4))
 (segment (start 133.284 89.8296) (end 132.8268 89.8296) (width 0.2) (layer "F.Cu") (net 4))
 (segment (start 130.0052 78.1986) (end 129.353558 78.850242) (width 0.2) (layer "F.Cu") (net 4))
 (segment (start 121.3358 94.361) (end 121.3612 94.3864) (width 0.2) (layer "F.Cu") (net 4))
 (segment (start 133.1454 88.355) (end 133.1454 88.319386) (width 0.2) (layer "F.Cu") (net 4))
 (segment (start 133.1454 88.355) (end 135.0704 90.28) (width 0.2) (layer "F.Cu") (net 4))
 (segment (start 132.6454 88.855) (end 133.1454 88.355) (width 0.2) (layer "F.Cu") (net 4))
 (segment (start 117.0686 89.5604) (end 122.6076 84.0214) (width 0.2) (layer "F.Cu") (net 4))
 (segment (start 121.3612 94.3864) (end 121.0056 94.0308) (width 0.2) (layer "F.Cu") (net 4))
 (segment (start 132.3176 78.1986) (end 130.0052 78.1986) (width 0.2) (layer "F.Cu") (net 4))
 (segment (start 135.0704 90.315614) (end 134.859786 90.105) (width 0.2) (layer "F.Cu") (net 4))
 (segment (start 135.1062 90.9424) (end 135.0704 90.9066) (width 0.2) (layer "F.Cu") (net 4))
 (segment (start 132.6454 90.805) (end 132.6454 88.855) (width 0.2) (layer "F.Cu") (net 4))
 (segment (start 118.8358 94.0308) (end 118.8358 91.3276) (width 0.2) (layer "F.Cu") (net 4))
 (segment (start 144.3736 81.3562) (end 144.3736 89.02444) (width 0.2) (layer "F.Cu") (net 4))
 (segment (start 135.0704 91.294386) (end 135.0704 90.9066) (width 0.2) (layer "F.Cu") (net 4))
 (segment (start 125.8358 95.7308) (end 124.8358 96.7308) (width 0.2) (layer "F.Cu") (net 4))
 (segment (start 142.517 90.28) (end 143.4812 89.3158) (width 0.2) (layer "F.Cu") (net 4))
 (segment (start 121.3358 94.0308) (end 121.3358 94.361) (width 0.2) (layer "F.Cu") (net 4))
 (segment (start 144.08224 89.3158) (end 143.4812 89.3158) (width 0.2) (layer "F.Cu") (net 4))
 (segment (start 135.1062 96.7238) (end 135.1062 90.9424) (width 0.2) (layer "F.Cu") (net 4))
 (segment (start 125.8358 94.0308) (end 125.8358 95.7308) (width 0.2) (layer "F.Cu") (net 4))
 (segment (start 133.5268 89.5868) (end 133.284 89.8296) (width 0.2) (layer "F.Cu") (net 4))
 (segment (start 117.6674 92.8624) (end 118.8358 94.0308) (width 0.2) (layer "F.Cu") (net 4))
 (via (at 127.5842 80.6196) (size 0.6) (drill 0.3) (layers "F.Cu" "B.Cu") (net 4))
 (via (at 120.985798 96.7308) (size 0.6) (drill 0.3) (layers "F.Cu" "B.Cu") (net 4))
 (via (at 121.3612 94.3864) (size 0.6) (drill 0.3) (layers "F.Cu" "B.Cu") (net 4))
 (via (at 120.1166 72.6186) (size 0.6) (drill 0.3) (layers "F.Cu" "B.Cu") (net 4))
 (via (at 122.6076 83.9986) (size 0.6) (drill 0.3) (layers "F.Cu" "B.Cu") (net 4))
 (via (at 129.353558 78.850242) (size 0.6) (drill 0.3) (layers "F.Cu" "B.Cu") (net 4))
 (segment (start 120.1166 72.6186) (end 120.1928 72.6948) (width 0.2) (layer "B.Cu") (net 4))
 (segment (start 123.848835 87.373) (end 122.937565 87.373) (width 0.2) (layer "B.Cu") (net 4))
 (segment (start 120.1928 72.6948) (end 120.1928 81.5838) (width 0.2) (layer "B.Cu") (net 4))
 (segment (start 120.1928 81.5838) (end 122.6076 83.9986) (width 0.2) (layer "B.Cu") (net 4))
 (segment (start 119.8358 96.7308) (end 120.985798 96.7308) (width 0.2) (layer "B.Cu") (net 4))
 (segment (start 124.4932 83.7106) (end 124.4932 86.728635) (width 0.2) (layer "B.Cu") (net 4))
 (segment (start 121.3612 94.3864) (end 121.3612 96.355398) (width 0.2) (layer "B.Cu") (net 4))
 (segment (start 129.353558 78.850242) (end 127.5842 80.6196) (width 0.2) (layer "B.Cu") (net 4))
 (segment (start 122.937565 87.373) (end 122.2932 86.728635) (width 0.2) (layer "B.Cu") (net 4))
 (segment (start 124.4932 86.728635) (end 123.848835 87.373) (width 0.2) (layer "B.Cu") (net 4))
 (segment (start 127.5842 80.6196) (end 124.4932 83.7106) (width 0.2) (layer "B.Cu") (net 4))
 (segment (start 122.2932 84.313) (end 122.6076 83.9986) (width 0.2) (layer "B.Cu") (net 4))
 (segment (start 121.3612 96.355398) (end 120.985798 96.7308) (width 0.2) (layer "B.Cu") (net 4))
 (segment (start 122.2932 86.728635) (end 122.2932 84.313) (width 0.2) (layer "B.Cu") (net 4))
 (segment (start 140.1076 72.0482) (end 140.208 72.1486) (width 0.2) (layer "F.Cu") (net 37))
 (segment (start 140.1076 71.9986) (end 140.1076 72.0482) (width 0.2) (layer "F.Cu") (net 37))
 (via (at 140.208 72.1486) (size 0.6) (drill 0.3) (layers "F.Cu" "B.Cu") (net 37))
 (segment (start 142.7562 88.19184) (end 142.88016 88.3158) (width 0.2) (layer "B.Cu") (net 37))
 (segment (start 140.208 72.1486) (end 140.208 80.250471) (width 0.2) (layer "B.Cu") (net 37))
 (segment (start 142.88016 88.3158) (end 143.4812 88.3158) (width 0.2) (layer "B.Cu") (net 37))
 (segment (start 142.7562 82.798671) (end 142.7562 88.19184) (width 0.2) (layer "B.Cu") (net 37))
 (segment (start 140.208 80.250471) (end 142.7562 82.798671) (width 0.2) (layer "B.Cu") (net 37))
 (segment (start 118.498494 71.3182) (end 118.8939 71.713606) (width 0.2) (layer "F.Cu") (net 5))
 (segment (start 127.4076 73.4986) (end 140.1076 73.4986) (width 0.2) (layer "F.Cu") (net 5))
 (segment (start 118.8939 71.713606) (end 118.8939 74.5849) (width 0.2) (layer "F.Cu") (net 5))
 (segment (start 117.0686 81.9604) (end 114.4939 79.3857) (width 0.2) (layer "F.Cu") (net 5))
 (segment (start 118.8939 74.5849) (end 121.5576 77.2486) (width 0.2) (layer "F.Cu") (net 5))
 (segment (start 121.5576 77.2486) (end 123.6576 77.2486) (width 0.2) (layer "F.Cu") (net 5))
 (segment (start 114.889306 71.3182) (end 118.498494 71.3182) (width 0.2) (layer "F.Cu") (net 5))
 (segment (start 114.4939 79.3857) (end 114.4939 71.713606) (width 0.2) (layer "F.Cu") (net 5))
 (segment (start 123.6576 77.2486) (end 127.4076 73.4986) (width 0.2) (layer "F.Cu") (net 5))
 (segment (start 114.4939 71.713606) (end 114.889306 71.3182) (width 0.2) (layer "F.Cu") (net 5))
 (segment (start 145.4576 71.057178) (end 145.399022 70.9986) (width 0.2) (layer "F.Cu") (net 35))
 (segment (start 144.3736 76.2762) (end 143.846 75.7486) (width 0.2) (layer "F.Cu") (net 35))
 (segment (start 121.1939 74.0261) (end 122.1664 74.9986) (width 0.2) (layer "F.Cu") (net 35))
 (segment (start 145.399022 70.9986) (end 121.908906 70.9986) (width 0.2) (layer "F.Cu") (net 35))
 (segment (start 122.1664 74.9986) (end 122.6076 74.9986) (width 0.2) (layer "F.Cu") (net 35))
 (segment (start 144.3736 76.2762) (end 145.4576 75.1922) (width 0.2) (layer "F.Cu") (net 35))
 (segment (start 121.1939 71.713606) (end 121.1939 74.0261) (width 0.2) (layer "F.Cu") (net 35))
 (segment (start 145.4576 75.1922) (end 145.4576 71.057178) (width 0.2) (layer "F.Cu") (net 35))
 (segment (start 121.908906 70.9986) (end 121.1939 71.713606) (width 0.2) (layer "F.Cu") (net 35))
 (segment (start 130.6954 88.855) (end 128.86 88.855) (width 0.2) (layer "F.Cu") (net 32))
 (segment (start 128.86 88.855) (end 128.857237 88.857763) (width 0.2) (layer "F.Cu") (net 32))
 (segment (start 140.1076 82.4986) (end 140.4076 82.4986) (width 0.2) (layer "F.Cu") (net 32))
 (segment (start 128.857237 88.857763) (end 128.857237 88.937923) (width 0.2) (layer "F.Cu") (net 32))
 (via (at 128.857237 88.937923) (size 0.6) (drill 0.3) (layers "F.Cu" "B.Cu") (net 32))
 (via (at 140.1076 82.4986) (size 0.6) (drill 0.3) (layers "F.Cu" "B.Cu") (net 32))
 (segment (start 133.668277 88.937923) (end 140.1076 82.4986) (width 0.2) (layer "B.Cu") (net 32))
 (segment (start 128.857237 88.937923) (end 133.668277 88.937923) (width 0.2) (layer "B.Cu") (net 32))
 (segment (start 130.6562 88.3158) (end 128.905 88.3158) (width 0.2) (layer "F.Cu") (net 31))
 (segment (start 140.1076 80.9986) (end 140.4076 80.9986) (width 0.2) (layer "F.Cu") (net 31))
 (segment (start 130.6954 88.355) (end 130.6562 88.3158) (width 0.2) (layer "F.Cu") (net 31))
 (segment (start 128.350093 88.3158) (end 128.258094 88.407799) (width 0.2) (layer "F.Cu") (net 31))
 (segment (start 128.905 88.3158) (end 128.350093 88.3158) (width 0.2) (layer "F.Cu") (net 31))
 (segment (start 128.905 88.3158) (end 129.0066 88.3158) (width 0.2) (layer "F.Cu") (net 31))
 (via (at 140.1076 80.9986) (size 0.6) (drill 0.3) (layers "F.Cu" "B.Cu") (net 31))
 (via (at 128.258094 88.407799) (size 0.6) (drill 0.3) (layers "F.Cu" "B.Cu") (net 31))
 (segment (start 128.258094 88.407799) (end 128.527893 88.138) (width 0.2) (layer "B.Cu") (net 31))
 (segment (start 132.9682 88.138) (end 140.1076 80.9986) (width 0.2) (layer "B.Cu") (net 31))
 (segment (start 128.527893 88.138) (end 132.9682 88.138) (width 0.2) (layer "B.Cu") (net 31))
 (segment (start 144.812 95.0468) (end 144.8562 95.0468) (width 0.2) (layer "F.Cu") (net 15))
 (segment (start 134.859786 85.205) (end 136.2954 86.640614) (width 0.2) (layer "F.Cu") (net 15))
 (segment (start 136.2954 89.569386) (end 136.009786 89.855) (width 0.2) (layer "F.Cu") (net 15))
 (segment (start 136.009786 89.855) (end 135.5954 89.855) (width 0.2) (layer "F.Cu") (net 15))
 (segment (start 121.6743 78.7486) (end 115.5439 72.6182) (width 0.2) (layer "F.Cu") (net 15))
 (segment (start 138.3792 89.8652) (end 138.3284 89.8144) (width 0.2) (layer "F.Cu") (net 15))
 (segment (start 144.8562 95.0468) (end 144.8816 95.0722) (width 0.2) (layer "F.Cu") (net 15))
 (segment (start 138.3284 89.8144) (end 138.3284 89.68) (width 0.2) (layer "F.Cu") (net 15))
 (segment (start 136.2954 86.640614) (end 128.403386 78.7486) (width 0.2) (layer "F.Cu") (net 15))
 (segment (start 138.083386 89.569386) (end 138.3792 89.8652) (width 0.2) (layer "F.Cu") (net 15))
 (segment (start 128.403386 78.7486) (end 121.6743 78.7486) (width 0.2) (layer "F.Cu") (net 15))
 (segment (start 136.2954 89.569386) (end 138.083386 89.569386) (width 0.2) (layer "F.Cu") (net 15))
 (segment (start 136.2954 86.640614) (end 136.2954 89.569386) (width 0.2) (layer "F.Cu") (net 15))
 (via (at 123.686887 97.1558) (size 0.6) (drill 0.3) (layers "F.Cu" "B.Cu") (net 15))
 (via (at 138.3284 89.68) (size 0.6) (drill 0.3) (layers "F.Cu" "B.Cu") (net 15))
 (via (at 144.8816 95.0722) (size 0.6) (drill 0.3) (layers "F.Cu" "B.Cu") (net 15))
 (segment (start 139.4894 89.68) (end 138.3284 89.68) (width 0.2) (layer "B.Cu") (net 15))
 (segment (start 138.3284 89.68) (end 130.2526 97.7558) (width 0.2) (layer "B.Cu") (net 15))
 (segment (start 144.8816 95.0722) (end 139.4894 89.68) (width 0.2) (layer "B.Cu") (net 15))
 (segment (start 124.286887 97.7558) (end 123.686887 97.1558) (width 0.2) (layer "B.Cu") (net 15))
 (segment (start 130.2526 97.7558) (end 124.286887 97.7558) (width 0.2) (layer "B.Cu") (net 15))
 (segment (start 133.1454 90.805) (end 133.1454 91.219386) (width 0.2) (layer "F.Cu") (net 11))
 (segment (start 122.4858 97.7558) (end 122.3358 97.6058) (width 0.2) (layer "F.Cu") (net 11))
 (segment (start 133.1454 91.219386) (end 126.608986 97.7558) (width 0.2) (layer "F.Cu") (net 11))
 (segment (start 122.3358 97.6058) (end 122.3358 96.7308) (width 0.2) (layer "F.Cu") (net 11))
 (segment (start 126.608986 97.7558) (end 122.4858 97.7558) (width 0.2) (layer "F.Cu") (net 11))
 (segment (start 133.6454 91.285072) (end 126.774672 98.1558) (width 0.2) (layer "F.Cu") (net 12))
 (segment (start 126.774672 98.1558) (end 119.811231 98.1558) (width 0.2) (layer "F.Cu") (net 12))
 (segment (start 122.9858 95.8558) (end 122.9858 96.7308) (width 0.2) (layer "F.Cu") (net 12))
 (segment (start 118.8108 97.155369) (end 118.8108 96.306231) (width 0.2) (layer "F.Cu") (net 12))
 (segment (start 118.8108 96.306231) (end 119.411231 95.7058) (width 0.2) (layer "F.Cu") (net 12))
 (segment (start 119.811231 98.1558) (end 118.8108 97.155369) (width 0.2) (layer "F.Cu") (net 12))
 (segment (start 133.6454 90.805) (end 133.6454 91.285072) (width 0.2) (layer "F.Cu") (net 12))
 (segment (start 122.8358 95.7058) (end 122.9858 95.8558) (width 0.2) (layer "F.Cu") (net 12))
 (segment (start 119.411231 95.7058) (end 122.8358 95.7058) (width 0.2) (layer "F.Cu") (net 12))
 (segment (start 147.135 96.7238) (end 148.812 95.0468) (width 0.2) (layer "F.Cu") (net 3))
 (segment (start 141.4062 96.7238) (end 147.135 96.7238) (width 0.2) (layer "F.Cu") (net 3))
 (segment (start 116.6872 89.9418) (end 116.785757 89.843243) (width 0.2) (layer "F.Cu") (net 6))
 (segment (start 116.6872 92.8624) (end 116.6872 89.9418) (width 0.2) (layer "F.Cu") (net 6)))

